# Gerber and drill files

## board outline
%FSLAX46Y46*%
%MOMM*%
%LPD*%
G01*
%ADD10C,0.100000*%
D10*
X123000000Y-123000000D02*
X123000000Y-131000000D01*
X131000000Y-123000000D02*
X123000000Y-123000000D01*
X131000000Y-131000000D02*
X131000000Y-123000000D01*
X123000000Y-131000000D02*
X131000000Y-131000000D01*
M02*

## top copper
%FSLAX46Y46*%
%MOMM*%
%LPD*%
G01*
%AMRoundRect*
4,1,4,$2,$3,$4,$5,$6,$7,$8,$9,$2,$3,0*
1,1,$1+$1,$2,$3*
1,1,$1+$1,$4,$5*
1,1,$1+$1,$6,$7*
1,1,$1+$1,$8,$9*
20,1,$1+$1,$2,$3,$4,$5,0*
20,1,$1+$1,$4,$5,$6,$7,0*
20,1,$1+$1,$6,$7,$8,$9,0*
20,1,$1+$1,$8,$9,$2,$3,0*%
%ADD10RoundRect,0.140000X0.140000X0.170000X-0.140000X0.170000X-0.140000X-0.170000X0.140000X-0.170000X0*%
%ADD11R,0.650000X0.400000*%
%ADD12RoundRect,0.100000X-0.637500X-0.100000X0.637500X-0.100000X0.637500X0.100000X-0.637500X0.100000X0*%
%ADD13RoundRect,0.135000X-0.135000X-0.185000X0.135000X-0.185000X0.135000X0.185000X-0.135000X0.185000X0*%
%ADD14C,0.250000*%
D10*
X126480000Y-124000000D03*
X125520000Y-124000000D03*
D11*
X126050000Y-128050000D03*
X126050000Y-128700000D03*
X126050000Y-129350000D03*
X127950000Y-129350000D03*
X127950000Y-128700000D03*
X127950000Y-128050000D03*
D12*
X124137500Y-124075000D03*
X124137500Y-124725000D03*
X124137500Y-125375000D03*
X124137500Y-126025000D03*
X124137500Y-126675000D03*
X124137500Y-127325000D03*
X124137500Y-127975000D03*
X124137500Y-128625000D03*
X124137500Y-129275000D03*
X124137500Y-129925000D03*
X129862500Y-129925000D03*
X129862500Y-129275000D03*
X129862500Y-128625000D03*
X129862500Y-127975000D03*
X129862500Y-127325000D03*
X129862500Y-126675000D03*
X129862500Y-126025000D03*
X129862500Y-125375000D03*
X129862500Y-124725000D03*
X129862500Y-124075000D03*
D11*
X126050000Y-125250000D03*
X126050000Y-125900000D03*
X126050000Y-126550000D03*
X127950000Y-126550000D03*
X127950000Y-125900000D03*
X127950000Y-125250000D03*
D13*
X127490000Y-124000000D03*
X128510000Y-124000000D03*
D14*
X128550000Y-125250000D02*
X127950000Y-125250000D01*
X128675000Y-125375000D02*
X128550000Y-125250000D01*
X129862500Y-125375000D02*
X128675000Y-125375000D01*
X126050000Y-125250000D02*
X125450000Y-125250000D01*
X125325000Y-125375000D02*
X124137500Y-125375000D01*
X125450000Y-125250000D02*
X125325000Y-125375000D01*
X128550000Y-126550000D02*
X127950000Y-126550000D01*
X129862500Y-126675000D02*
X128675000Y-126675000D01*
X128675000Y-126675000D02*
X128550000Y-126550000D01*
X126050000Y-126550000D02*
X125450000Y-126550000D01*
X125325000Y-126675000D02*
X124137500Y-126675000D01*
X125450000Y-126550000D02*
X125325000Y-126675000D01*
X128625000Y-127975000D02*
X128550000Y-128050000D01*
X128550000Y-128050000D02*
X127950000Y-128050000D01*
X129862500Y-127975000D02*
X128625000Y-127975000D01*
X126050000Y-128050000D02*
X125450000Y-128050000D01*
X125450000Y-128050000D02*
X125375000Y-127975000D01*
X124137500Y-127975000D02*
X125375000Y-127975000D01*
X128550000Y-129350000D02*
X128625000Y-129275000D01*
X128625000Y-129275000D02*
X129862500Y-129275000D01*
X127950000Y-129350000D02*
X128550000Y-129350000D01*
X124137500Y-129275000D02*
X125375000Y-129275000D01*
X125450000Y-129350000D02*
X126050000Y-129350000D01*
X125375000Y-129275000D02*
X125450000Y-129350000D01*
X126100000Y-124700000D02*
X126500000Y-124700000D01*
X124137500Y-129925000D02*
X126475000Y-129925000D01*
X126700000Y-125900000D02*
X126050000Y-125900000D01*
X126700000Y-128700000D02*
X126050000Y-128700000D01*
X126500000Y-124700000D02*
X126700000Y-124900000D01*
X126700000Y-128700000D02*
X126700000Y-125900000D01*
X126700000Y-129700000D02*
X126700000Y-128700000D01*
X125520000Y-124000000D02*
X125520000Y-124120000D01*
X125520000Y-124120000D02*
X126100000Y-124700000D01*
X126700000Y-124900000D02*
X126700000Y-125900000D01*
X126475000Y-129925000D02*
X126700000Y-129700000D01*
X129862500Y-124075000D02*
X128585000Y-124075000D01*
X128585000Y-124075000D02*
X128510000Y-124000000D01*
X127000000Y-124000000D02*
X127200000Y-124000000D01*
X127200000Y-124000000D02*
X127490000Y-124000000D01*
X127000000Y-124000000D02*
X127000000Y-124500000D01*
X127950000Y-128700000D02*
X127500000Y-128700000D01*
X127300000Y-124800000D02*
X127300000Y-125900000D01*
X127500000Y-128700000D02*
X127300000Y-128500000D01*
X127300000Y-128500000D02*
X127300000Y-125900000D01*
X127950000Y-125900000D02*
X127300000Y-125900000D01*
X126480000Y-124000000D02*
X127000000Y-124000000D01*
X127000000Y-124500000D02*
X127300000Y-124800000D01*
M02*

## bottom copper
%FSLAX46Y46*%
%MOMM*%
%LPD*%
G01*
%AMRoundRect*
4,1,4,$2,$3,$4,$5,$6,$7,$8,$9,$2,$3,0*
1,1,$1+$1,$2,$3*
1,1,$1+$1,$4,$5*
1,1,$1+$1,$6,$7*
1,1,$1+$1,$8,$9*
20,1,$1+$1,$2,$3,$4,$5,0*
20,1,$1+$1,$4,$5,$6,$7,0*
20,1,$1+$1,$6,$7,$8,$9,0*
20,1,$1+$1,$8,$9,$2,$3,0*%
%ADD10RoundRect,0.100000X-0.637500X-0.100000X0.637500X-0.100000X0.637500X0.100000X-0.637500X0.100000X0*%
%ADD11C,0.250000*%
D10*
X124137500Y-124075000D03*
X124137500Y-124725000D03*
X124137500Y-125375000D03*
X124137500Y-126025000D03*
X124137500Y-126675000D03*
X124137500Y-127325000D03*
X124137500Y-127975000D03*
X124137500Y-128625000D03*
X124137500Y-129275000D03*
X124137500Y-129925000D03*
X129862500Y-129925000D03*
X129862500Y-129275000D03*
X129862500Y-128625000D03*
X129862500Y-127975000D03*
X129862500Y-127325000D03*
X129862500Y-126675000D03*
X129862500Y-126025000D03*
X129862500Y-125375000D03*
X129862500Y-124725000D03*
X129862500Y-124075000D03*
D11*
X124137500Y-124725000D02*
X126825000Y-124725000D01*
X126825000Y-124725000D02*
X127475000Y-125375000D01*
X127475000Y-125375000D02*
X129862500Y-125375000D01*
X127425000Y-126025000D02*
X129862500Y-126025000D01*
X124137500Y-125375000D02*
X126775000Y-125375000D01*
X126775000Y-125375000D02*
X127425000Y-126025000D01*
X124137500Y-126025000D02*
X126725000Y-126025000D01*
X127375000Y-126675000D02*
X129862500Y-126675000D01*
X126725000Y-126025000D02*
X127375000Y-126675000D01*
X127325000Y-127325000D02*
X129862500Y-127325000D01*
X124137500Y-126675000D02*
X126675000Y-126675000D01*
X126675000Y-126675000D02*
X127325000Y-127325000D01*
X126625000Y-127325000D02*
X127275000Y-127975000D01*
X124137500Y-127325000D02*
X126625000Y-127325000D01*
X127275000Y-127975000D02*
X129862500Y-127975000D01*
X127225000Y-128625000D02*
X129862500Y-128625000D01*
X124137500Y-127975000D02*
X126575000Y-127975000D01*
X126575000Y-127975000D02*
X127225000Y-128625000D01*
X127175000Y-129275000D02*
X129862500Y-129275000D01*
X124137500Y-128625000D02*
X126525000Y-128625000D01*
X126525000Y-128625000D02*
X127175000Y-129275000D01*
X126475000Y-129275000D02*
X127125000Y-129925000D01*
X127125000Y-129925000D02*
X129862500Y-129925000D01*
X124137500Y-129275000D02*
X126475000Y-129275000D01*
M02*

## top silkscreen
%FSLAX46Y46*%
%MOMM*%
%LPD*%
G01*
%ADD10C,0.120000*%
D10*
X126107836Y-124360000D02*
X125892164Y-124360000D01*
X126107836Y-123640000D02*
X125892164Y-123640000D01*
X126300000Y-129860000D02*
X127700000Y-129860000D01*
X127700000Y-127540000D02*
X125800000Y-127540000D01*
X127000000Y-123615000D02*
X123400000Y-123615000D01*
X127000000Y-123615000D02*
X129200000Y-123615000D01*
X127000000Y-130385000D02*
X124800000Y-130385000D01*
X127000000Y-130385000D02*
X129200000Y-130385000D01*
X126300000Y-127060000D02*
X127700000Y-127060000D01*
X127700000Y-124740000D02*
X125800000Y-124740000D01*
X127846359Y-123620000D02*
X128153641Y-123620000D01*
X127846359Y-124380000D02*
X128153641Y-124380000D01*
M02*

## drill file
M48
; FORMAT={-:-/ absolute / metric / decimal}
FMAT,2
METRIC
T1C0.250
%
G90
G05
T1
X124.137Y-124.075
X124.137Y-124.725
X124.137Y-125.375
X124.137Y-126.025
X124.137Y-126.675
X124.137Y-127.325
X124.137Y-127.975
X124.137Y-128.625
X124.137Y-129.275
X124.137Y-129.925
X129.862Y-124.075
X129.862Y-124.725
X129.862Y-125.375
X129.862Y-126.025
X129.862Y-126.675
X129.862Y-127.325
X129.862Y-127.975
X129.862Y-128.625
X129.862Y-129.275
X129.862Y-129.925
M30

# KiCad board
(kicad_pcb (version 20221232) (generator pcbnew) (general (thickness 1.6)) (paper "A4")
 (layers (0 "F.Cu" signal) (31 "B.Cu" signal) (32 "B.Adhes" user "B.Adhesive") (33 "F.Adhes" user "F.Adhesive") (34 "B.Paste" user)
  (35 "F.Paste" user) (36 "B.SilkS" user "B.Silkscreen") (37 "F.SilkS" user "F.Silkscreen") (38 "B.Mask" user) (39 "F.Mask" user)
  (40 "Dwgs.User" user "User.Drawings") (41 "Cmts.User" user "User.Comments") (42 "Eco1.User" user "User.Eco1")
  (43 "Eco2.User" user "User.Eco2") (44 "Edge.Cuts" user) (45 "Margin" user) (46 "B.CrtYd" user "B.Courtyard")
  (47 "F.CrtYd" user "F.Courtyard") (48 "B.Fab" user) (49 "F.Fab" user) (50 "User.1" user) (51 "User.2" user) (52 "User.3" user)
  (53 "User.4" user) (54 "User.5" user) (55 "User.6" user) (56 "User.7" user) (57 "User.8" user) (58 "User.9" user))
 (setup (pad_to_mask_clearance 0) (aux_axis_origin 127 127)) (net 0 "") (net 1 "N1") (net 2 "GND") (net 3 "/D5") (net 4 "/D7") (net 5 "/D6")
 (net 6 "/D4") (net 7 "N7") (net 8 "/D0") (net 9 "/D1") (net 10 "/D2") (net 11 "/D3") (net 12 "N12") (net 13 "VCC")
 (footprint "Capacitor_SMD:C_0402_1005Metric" (layer "F.Cu") (at 126 124 180)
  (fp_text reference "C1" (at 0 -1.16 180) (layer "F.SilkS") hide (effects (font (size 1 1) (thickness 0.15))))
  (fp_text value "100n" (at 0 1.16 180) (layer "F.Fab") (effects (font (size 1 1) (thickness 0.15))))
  (fp_line (start -0.107836 -0.36) (end 0.107836 -0.36) (stroke (width 0.12) (type solid)) (layer "F.SilkS"))
  (fp_line (start -0.107836 0.36) (end 0.107836 0.36) (stroke (width 0.12) (type solid)) (layer "F.SilkS"))
  (pad "1" smd roundrect locked (at -0.48 0 180) (size 0.56 0.62) (layers "F.Cu" "F.Paste" "F.Mask") (roundrect_rratio 0.25) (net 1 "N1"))
  (pad "2" smd roundrect locked (at 0.48 0 180) (size 0.56 0.62) (layers "F.Cu" "F.Paste" "F.Mask") (roundrect_rratio 0.25) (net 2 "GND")))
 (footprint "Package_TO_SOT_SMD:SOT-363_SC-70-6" (layer "F.Cu") (at 127 128.7)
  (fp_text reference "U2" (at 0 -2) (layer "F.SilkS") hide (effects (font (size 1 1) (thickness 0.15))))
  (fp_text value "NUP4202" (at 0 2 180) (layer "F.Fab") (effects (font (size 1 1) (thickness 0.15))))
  (fp_line (start -0.7 1.16) (end 0.7 1.16) (stroke (width 0.12) (type solid)) (layer "F.SilkS"))
  (fp_line (start 0.7 -1.16) (end -1.2 -1.16) (stroke (width 0.12) (type solid)) (layer "F.SilkS"))
  (pad "1" smd rect locked (at -0.95 -0.65) (size 0.65 0.4) (layers "F.Cu" "F.Paste" "F.Mask") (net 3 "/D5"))
  (pad "2" smd rect locked (at -0.95 0) (size 0.65 0.4) (layers "F.Cu" "F.Paste" "F.Mask") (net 2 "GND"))
  (pad "3" smd rect locked (at -0.95 0.65) (size 0.65 0.4) (layers "F.Cu" "F.Paste" "F.Mask") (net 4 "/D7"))
  (pad "4" smd rect locked (at 0.95 0.65) (size 0.65 0.4) (layers "F.Cu" "F.Paste" "F.Mask") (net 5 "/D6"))
  (pad "5" smd rect locked (at 0.95 0) (size 0.65 0.4) (layers "F.Cu" "F.Paste" "F.Mask") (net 1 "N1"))
  (pad "6" smd rect locked (at 0.95 -0.65) (size 0.65 0.4) (layers "F.Cu" "F.Paste" "F.Mask") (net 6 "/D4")))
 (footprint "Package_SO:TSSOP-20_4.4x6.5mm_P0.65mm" (layer "F.Cu") (at 127 127)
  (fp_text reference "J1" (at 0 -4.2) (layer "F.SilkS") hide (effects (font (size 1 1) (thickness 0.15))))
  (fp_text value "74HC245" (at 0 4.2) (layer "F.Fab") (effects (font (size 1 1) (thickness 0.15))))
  (fp_line (start 0 -3.385) (end -3.6 -3.385) (stroke (width 0.12) (type solid)) (layer "F.SilkS"))
  (fp_line (start 0 -3.385) (end 2.2 -3.385) (stroke (width 0.12) (type solid)) (layer "F.SilkS"))
  (fp_line (start 0 3.385) (end -2.2 3.385) (stroke (width 0.12) (type solid)) (layer "F.SilkS"))
  (fp_line (start 0 3.385) (end 2.2 3.385) (stroke (width 0.12) (type solid)) (layer "F.SilkS"))
  (pad "1" thru_hole roundrect (at -2.8625 -2.925) (size 1.475 0.4) (drill 0.25) (layers *.Cu *.Mask) (roundrect_rratio 0.25) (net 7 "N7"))
  (pad "2" thru_hole roundrect (at -2.8625 -2.275) (size 1.475 0.4) (drill 0.25) (layers *.Cu *.Mask) (roundrect_rratio 0.25) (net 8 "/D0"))
  (pad "3" thru_hole roundrect (at -2.8625 -1.625) (size 1.475 0.4) (drill 0.25) (layers *.Cu *.Mask) (roundrect_rratio 0.25) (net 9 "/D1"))
  (pad "4" thru_hole roundrect (at -2.8625 -0.975) (size 1.475 0.4) (drill 0.25) (layers *.Cu *.Mask) (roundrect_rratio 0.25) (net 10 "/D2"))
  (pad "5" thru_hole roundrect (at -2.8625 -0.325) (size 1.475 0.4) (drill 0.25) (layers *.Cu *.Mask) (roundrect_rratio 0.25) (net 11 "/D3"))
  (pad "6" thru_hole roundrect (at -2.8625 0.325) (size 1.475 0.4) (drill 0.25) (layers *.Cu *.Mask) (roundrect_rratio 0.25) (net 6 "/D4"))
  (pad "7" thru_hole roundrect (at -2.8625 0.975) (size 1.475 0.4) (drill 0.25) (layers *.Cu *.Mask) (roundrect_rratio 0.25) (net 3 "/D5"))
  (pad "8" thru_hole roundrect (at -2.8625 1.625) (size 1.475 0.4) (drill 0.25) (layers *.Cu *.Mask) (roundrect_rratio 0.25) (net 5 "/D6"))
  (pad "9" thru_hole roundrect (at -2.8625 2.275) (size 1.475 0.4) (drill 0.25) (layers *.Cu *.Mask) (roundrect_rratio 0.25) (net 4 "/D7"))
  (pad "10" thru_hole roundrect (at -2.8625 2.925) (size 1.475 0.4) (drill 0.25) (layers *.Cu *.Mask) (roundrect_rratio 0.25) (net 2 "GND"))
  (pad "11" thru_hole roundrect (at 2.8625 2.925) (size 1.475 0.4) (drill 0.25) (layers *.Cu *.Mask) (roundrect_rratio 0.25) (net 4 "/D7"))
  (pad "12" thru_hole roundrect (at 2.8625 2.275) (size 1.475 0.4) (drill 0.25) (layers *.Cu *.Mask) (roundrect_rratio 0.25) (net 5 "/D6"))
  (pad "13" thru_hole roundrect (at 2.8625 1.625) (size 1.475 0.4) (drill 0.25) (layers *.Cu *.Mask) (roundrect_rratio 0.25) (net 3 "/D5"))
  (pad "14" thru_hole roundrect (at 2.8625 0.975) (size 1.475 0.4) (drill 0.25) (layers *.Cu *.Mask) (roundrect_rratio 0.25) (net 6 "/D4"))
  (pad "15" thru_hole roundrect (at 2.8625 0.325) (size 1.475 0.4) (drill 0.25) (layers *.Cu *.Mask) (roundrect_rratio 0.25) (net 11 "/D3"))
  (pad "16" thru_hole roundrect (at 2.8625 -0.325) (size 1.475 0.4) (drill 0.25) (layers *.Cu *.Mask) (roundrect_rratio 0.25) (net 10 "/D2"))
  (pad "17" thru_hole roundrect (at 2.8625 -0.975) (size 1.475 0.4) (drill 0.25) (layers *.Cu *.Mask) (roundrect_rratio 0.25) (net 9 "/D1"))
  (pad "18" thru_hole roundrect (at 2.8625 -1.625) (size 1.475 0.4) (drill 0.25) (layers *.Cu *.Mask) (roundrect_rratio 0.25) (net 8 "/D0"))
  (pad "19" thru_hole roundrect (at 2.8625 -2.275) (size 1.475 0.4) (drill 0.25) (layers *.Cu *.Mask) (roundrect_rratio 0.25) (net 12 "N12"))
  (pad "20" thru_hole roundrect (at 2.8625 -2.925) (size 1.475 0.4) (drill 0.25) (layers *.Cu *.Mask) (roundrect_rratio 0.25) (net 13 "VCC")))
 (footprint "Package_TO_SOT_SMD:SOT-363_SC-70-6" (layer "F.Cu") (at 127 125.9)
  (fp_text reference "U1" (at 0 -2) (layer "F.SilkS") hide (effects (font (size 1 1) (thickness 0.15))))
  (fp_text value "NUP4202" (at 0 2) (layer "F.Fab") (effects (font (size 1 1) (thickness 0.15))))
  (fp_line (start -0.7 1.16) (end 0.7 1.16) (stroke (width 0.12) (type solid)) (layer "F.SilkS"))
  (fp_line (start 0.7 -1.16) (end -1.2 -1.16) (stroke (width 0.12) (type solid)) (layer "F.SilkS"))
  (pad "1" smd rect locked (at -0.95 -0.65) (size 0.65 0.4) (layers "F.Cu" "F.Paste" "F.Mask") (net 9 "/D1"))
  (pad "2" smd rect locked (at -0.95 0) (size 0.65 0.4) (layers "F.Cu" "F.Paste" "F.Mask") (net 2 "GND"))
  (pad "3" smd rect locked (at -0.95 0.65) (size 0.65 0.4) (layers "F.Cu" "F.Paste" "F.Mask") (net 11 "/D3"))
  (pad "4" smd rect locked (at 0.95 0.65) (size 0.65 0.4) (layers "F.Cu" "F.Paste" "F.Mask") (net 10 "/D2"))
  (pad "5" smd rect locked (at 0.95 0) (size 0.65 0.4) (layers "F.Cu" "F.Paste" "F.Mask") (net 1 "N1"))
  (pad "6" smd rect locked (at 0.95 -0.65) (size 0.65 0.4) (layers "F.Cu" "F.Paste" "F.Mask") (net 8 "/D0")))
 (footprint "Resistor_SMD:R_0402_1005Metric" (layer "F.Cu") (at 128 124)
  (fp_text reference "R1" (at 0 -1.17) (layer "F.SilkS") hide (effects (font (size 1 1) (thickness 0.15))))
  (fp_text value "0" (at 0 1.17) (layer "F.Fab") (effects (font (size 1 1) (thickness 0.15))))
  (fp_line (start -0.153641 -0.38) (end 0.153641 -0.38) (stroke (width 0.12) (type solid)) (layer "F.SilkS"))
  (fp_line (start -0.153641 0.38) (end 0.153641 0.38) (stroke (width 0.12) (type solid)) (layer "F.SilkS"))
  (pad "1" smd roundrect locked (at -0.51 0) (size 0.54 0.64) (layers "F.Cu" "F.Paste" "F.Mask") (roundrect_rratio 0.25) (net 1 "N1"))
  (pad "2" smd roundrect locked (at 0.51 0) (size 0.54 0.64) (layers "F.Cu" "F.Paste" "F.Mask") (roundrect_rratio 0.25) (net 13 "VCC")))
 (gr_line (start 123 123) (end 123 131) (stroke (width 0.1) (type default)) (layer "Edge.Cuts"))
 (gr_line (start 131 123) (end 123 123) (stroke (width 0.1) (type default)) (layer "Edge.Cuts"))
 (gr_line (start 131 131) (end 131 123) (stroke (width 0.1) (type default)) (layer "Edge.Cuts"))
 (gr_line (start 123 131) (end 131 131) (stroke (width 0.1) (type default)) (layer "Edge.Cuts"))
 (segment (start 128.55 125.25) (end 127.95 125.25) (width 0.25) (layer "F.Cu") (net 8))
 (segment (start 128.675 125.375) (end 128.55 125.25) (width 0.25) (layer "F.Cu") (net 8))
 (segment (start 129.8625 125.375) (end 128.675 125.375) (width 0.25) (layer "F.Cu") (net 8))
 (segment (start 124.1375 124.725) (end 126.825 124.725) (width 0.25) (layer "B.Cu") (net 8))
 (segment (start 126.825 124.725) (end 127.475 125.375) (width 0.25) (layer "B.Cu") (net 8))
 (segment (start 127.475 125.375) (end 129.8625 125.375) (width 0.25) (layer "B.Cu") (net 8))
 (segment (start 126.05 125.25) (end 125.45 125.25) (width 0.25) (layer "F.Cu") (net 9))
 (segment (start 125.325 125.375) (end 124.1375 125.375) (width 0.25) (layer "F.Cu") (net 9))
 (segment (start 125.45 125.25) (end 125.325 125.375) (width 0.25) (layer "F.Cu") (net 9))
 (segment (start 127.425 126.025) (end 129.8625 126.025) (width 0.25) (layer "B.Cu") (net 9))
 (segment (start 124.1375 125.375) (end 126.775 125.375) (width 0.25) (layer "B.Cu") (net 9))
 (segment (start 126.775 125.375) (end 127.425 126.025) (width 0.25) (layer "B.Cu") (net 9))
 (segment (start 128.55 126.55) (end 127.95 126.55) (width 0.25) (layer "F.Cu") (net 10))
 (segment (start 129.8625 126.675) (end 128.675 126.675) (width 0.25) (layer "F.Cu") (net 10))
 (segment (start 128.675 126.675) (end 128.55 126.55) (width 0.25) (layer "F.Cu") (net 10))
 (segment (start 124.1375 126.025) (end 126.725 126.025) (width 0.25) (layer "B.Cu") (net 10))
 (segment (start 127.375 126.675) (end 129.8625 126.675) (width 0.25) (layer "B.Cu") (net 10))
 (segment (start 126.725 126.025) (end 127.375 126.675) (width 0.25) (layer "B.Cu") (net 10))
 (segment (start 126.05 126.55) (end 125.45 126.55) (width 0.25) (layer "F.Cu") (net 11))
 (segment (start 125.325 126.675) (end 124.1375 126.675) (width 0.25) (layer "F.Cu") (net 11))
 (segment (start 125.45 126.55) (end 125.325 126.675) (width 0.25) (layer "F.Cu") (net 11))
 (segment (start 127.325 127.325) (end 129.8625 127.325) (width 0.25) (layer "B.Cu") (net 11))
 (segment (start 124.1375 126.675) (end 126.675 126.675) (width 0.25) (layer "B.Cu") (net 11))
 (segment (start 126.675 126.675) (end 127.325 127.325) (width 0.25) (layer "B.Cu") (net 11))
 (segment (start 128.625 127.975) (end 128.55 128.05) (width 0.25) (layer "F.Cu") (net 6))
 (segment (start 128.55 128.05) (end 127.95 128.05) (width 0.25) (layer "F.Cu") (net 6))
 (segment (start 129.8625 127.975) (end 128.625 127.975) (width 0.25) (layer "F.Cu") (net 6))
 (segment (start 126.625 127.325) (end 127.275 127.975) (width 0.25) (layer "B.Cu") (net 6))
 (segment (start 124.1375 127.325) (end 126.625 127.325) (width 0.25) (layer "B.Cu") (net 6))
 (segment (start 127.275 127.975) (end 129.8625 127.975) (width 0.25) (layer "B.Cu") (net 6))
 (segment (start 126.05 128.05) (end 125.45 128.05) (width 0.25) (layer "F.Cu") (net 3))
 (segment (start 125.45 128.05) (end 125.375 127.975) (width 0.25) (layer "F.Cu") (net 3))
 (segment (start 124.1375 127.975) (end 125.375 127.975) (width 0.25) (layer "F.Cu") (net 3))
 (segment (start 127.225 128.625) (end 129.8625 128.625) (width 0.25) (layer "B.Cu") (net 3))
 (segment (start 124.1375 127.975) (end 126.575 127.975) (width 0.25) (layer "B.Cu") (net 3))
 (segment (start 126.575 127.975) (end 127.225 128.625) (width 0.25) (layer "B.Cu") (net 3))
 (segment (start 128.55 129.35) (end 128.625 129.275) (width 0.25) (layer "F.Cu") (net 5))
 (segment (start 128.625 129.275) (end 129.8625 129.275) (width 0.25) (layer "F.Cu") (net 5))
 (segment (start 127.95 129.35) (end 128.55 129.35) (width 0.25) (layer "F.Cu") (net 5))
 (segment (start 127.175 129.275) (end 129.8625 129.275) (width 0.25) (layer "B.Cu") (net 5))
 (segment (start 124.1375 128.625) (end 126.525 128.625) (width 0.25) (layer "B.Cu") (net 5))
 (segment (start 126.525 128.625) (end 127.175 129.275) (width 0.25) (layer "B.Cu") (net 5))
 (segment (start 124.1375 129.275) (end 125.375 129.275) (width 0.25) (layer "F.Cu") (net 4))
 (segment (start 125.45 129.35) (end 126.05 129.35) (width 0.25) (layer "F.Cu") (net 4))
 (segment (start 125.375 129.275) (end 125.45 129.35) (width 0.25) (layer "F.Cu") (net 4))
 (segment (start 126.475 129.275) (end 127.125 129.925) (width 0.25) (layer "B.Cu") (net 4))
 (segment (start 127.125 129.925) (end 129.8625 129.925) (width 0.25) (layer "B.Cu") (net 4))
 (segment (start 124.1375 129.275) (end 126.475 129.275) (width 0.25) (layer "B.Cu") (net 4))
 (segment (start 126.1 124.7) (end 126.5 124.7) (width 0.25) (layer "F.Cu") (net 2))
 (segment (start 124.1375 129.925) (end 126.475 129.925) (width 0.25) (layer "F.Cu") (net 2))
 (segment (start 126.7 125.9) (end 126.05 125.9) (width 0.25) (layer "F.Cu") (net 2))
 (segment (start 126.7 128.7) (end 126.05 128.7) (width 0.25) (layer "F.Cu") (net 2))
 (segment (start 126.5 124.7) (end 126.7 124.9) (width 0.25) (layer "F.Cu") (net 2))
 (segment (start 126.7 128.7) (end 126.7 125.9) (width 0.25) (layer "F.Cu") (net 2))
 (segment (start 126.7 129.7) (end 126.7 128.7) (width 0.25) (layer "F.Cu") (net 2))
 (segment (start 125.52 124) (end 125.52 124.12) (width 0.25) (layer "F.Cu") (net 2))
 (segment (start 125.52 124.12) (end 126.1 124.7) (width 0.25) (layer "F.Cu") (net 2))
 (segment (start 126.7 124.9) (end 126.7 125.9) (width 0.25) (layer "F.Cu") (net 2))
 (segment (start 126.475 129.925) (end 126.7 129.7) (width 0.25) (layer "F.Cu") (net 2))
 (segment (start 129.8625 124.075) (end 128.585 124.075) (width 0.25) (layer "F.Cu") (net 13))
 (segment (start 128.585 124.075) (end 128.51 124) (width 0.25) (layer "F.Cu") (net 13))
 (segment (start 127 124) (end 127.2 124) (width 0.25) (layer "F.Cu") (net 1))
 (segment (start 127.2 124) (end 127.49 124) (width 0.25) (layer "F.Cu") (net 1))
 (segment (start 127 124) (end 127 124.5) (width 0.25) (layer "F.Cu") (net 1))
 (segment (start 127.95 128.7) (end 127.5 128.7) (width 0.25) (layer "F.Cu") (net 1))
 (segment (start 127.3 124.8) (end 127.3 125.9) (width 0.25) (layer "F.Cu") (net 1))
 (segment (start 127.5 128.7) (end 127.3 128.5) (width 0.25) (layer "F.Cu") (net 1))
 (segment (start 127.3 128.5) (end 127.3 125.9) (width 0.25) (layer "F.Cu") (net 1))
 (segment (start 127.95 125.9) (end 127.3 125.9) (width 0.25) (layer "F.Cu") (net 1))
 (segment (start 126.48 124) (end 127 124) (width 0.25) (layer "F.Cu") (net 1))
 (segment (start 127 124.5) (end 127.3 124.8) (width 0.25) (layer "F.Cu") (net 1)))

